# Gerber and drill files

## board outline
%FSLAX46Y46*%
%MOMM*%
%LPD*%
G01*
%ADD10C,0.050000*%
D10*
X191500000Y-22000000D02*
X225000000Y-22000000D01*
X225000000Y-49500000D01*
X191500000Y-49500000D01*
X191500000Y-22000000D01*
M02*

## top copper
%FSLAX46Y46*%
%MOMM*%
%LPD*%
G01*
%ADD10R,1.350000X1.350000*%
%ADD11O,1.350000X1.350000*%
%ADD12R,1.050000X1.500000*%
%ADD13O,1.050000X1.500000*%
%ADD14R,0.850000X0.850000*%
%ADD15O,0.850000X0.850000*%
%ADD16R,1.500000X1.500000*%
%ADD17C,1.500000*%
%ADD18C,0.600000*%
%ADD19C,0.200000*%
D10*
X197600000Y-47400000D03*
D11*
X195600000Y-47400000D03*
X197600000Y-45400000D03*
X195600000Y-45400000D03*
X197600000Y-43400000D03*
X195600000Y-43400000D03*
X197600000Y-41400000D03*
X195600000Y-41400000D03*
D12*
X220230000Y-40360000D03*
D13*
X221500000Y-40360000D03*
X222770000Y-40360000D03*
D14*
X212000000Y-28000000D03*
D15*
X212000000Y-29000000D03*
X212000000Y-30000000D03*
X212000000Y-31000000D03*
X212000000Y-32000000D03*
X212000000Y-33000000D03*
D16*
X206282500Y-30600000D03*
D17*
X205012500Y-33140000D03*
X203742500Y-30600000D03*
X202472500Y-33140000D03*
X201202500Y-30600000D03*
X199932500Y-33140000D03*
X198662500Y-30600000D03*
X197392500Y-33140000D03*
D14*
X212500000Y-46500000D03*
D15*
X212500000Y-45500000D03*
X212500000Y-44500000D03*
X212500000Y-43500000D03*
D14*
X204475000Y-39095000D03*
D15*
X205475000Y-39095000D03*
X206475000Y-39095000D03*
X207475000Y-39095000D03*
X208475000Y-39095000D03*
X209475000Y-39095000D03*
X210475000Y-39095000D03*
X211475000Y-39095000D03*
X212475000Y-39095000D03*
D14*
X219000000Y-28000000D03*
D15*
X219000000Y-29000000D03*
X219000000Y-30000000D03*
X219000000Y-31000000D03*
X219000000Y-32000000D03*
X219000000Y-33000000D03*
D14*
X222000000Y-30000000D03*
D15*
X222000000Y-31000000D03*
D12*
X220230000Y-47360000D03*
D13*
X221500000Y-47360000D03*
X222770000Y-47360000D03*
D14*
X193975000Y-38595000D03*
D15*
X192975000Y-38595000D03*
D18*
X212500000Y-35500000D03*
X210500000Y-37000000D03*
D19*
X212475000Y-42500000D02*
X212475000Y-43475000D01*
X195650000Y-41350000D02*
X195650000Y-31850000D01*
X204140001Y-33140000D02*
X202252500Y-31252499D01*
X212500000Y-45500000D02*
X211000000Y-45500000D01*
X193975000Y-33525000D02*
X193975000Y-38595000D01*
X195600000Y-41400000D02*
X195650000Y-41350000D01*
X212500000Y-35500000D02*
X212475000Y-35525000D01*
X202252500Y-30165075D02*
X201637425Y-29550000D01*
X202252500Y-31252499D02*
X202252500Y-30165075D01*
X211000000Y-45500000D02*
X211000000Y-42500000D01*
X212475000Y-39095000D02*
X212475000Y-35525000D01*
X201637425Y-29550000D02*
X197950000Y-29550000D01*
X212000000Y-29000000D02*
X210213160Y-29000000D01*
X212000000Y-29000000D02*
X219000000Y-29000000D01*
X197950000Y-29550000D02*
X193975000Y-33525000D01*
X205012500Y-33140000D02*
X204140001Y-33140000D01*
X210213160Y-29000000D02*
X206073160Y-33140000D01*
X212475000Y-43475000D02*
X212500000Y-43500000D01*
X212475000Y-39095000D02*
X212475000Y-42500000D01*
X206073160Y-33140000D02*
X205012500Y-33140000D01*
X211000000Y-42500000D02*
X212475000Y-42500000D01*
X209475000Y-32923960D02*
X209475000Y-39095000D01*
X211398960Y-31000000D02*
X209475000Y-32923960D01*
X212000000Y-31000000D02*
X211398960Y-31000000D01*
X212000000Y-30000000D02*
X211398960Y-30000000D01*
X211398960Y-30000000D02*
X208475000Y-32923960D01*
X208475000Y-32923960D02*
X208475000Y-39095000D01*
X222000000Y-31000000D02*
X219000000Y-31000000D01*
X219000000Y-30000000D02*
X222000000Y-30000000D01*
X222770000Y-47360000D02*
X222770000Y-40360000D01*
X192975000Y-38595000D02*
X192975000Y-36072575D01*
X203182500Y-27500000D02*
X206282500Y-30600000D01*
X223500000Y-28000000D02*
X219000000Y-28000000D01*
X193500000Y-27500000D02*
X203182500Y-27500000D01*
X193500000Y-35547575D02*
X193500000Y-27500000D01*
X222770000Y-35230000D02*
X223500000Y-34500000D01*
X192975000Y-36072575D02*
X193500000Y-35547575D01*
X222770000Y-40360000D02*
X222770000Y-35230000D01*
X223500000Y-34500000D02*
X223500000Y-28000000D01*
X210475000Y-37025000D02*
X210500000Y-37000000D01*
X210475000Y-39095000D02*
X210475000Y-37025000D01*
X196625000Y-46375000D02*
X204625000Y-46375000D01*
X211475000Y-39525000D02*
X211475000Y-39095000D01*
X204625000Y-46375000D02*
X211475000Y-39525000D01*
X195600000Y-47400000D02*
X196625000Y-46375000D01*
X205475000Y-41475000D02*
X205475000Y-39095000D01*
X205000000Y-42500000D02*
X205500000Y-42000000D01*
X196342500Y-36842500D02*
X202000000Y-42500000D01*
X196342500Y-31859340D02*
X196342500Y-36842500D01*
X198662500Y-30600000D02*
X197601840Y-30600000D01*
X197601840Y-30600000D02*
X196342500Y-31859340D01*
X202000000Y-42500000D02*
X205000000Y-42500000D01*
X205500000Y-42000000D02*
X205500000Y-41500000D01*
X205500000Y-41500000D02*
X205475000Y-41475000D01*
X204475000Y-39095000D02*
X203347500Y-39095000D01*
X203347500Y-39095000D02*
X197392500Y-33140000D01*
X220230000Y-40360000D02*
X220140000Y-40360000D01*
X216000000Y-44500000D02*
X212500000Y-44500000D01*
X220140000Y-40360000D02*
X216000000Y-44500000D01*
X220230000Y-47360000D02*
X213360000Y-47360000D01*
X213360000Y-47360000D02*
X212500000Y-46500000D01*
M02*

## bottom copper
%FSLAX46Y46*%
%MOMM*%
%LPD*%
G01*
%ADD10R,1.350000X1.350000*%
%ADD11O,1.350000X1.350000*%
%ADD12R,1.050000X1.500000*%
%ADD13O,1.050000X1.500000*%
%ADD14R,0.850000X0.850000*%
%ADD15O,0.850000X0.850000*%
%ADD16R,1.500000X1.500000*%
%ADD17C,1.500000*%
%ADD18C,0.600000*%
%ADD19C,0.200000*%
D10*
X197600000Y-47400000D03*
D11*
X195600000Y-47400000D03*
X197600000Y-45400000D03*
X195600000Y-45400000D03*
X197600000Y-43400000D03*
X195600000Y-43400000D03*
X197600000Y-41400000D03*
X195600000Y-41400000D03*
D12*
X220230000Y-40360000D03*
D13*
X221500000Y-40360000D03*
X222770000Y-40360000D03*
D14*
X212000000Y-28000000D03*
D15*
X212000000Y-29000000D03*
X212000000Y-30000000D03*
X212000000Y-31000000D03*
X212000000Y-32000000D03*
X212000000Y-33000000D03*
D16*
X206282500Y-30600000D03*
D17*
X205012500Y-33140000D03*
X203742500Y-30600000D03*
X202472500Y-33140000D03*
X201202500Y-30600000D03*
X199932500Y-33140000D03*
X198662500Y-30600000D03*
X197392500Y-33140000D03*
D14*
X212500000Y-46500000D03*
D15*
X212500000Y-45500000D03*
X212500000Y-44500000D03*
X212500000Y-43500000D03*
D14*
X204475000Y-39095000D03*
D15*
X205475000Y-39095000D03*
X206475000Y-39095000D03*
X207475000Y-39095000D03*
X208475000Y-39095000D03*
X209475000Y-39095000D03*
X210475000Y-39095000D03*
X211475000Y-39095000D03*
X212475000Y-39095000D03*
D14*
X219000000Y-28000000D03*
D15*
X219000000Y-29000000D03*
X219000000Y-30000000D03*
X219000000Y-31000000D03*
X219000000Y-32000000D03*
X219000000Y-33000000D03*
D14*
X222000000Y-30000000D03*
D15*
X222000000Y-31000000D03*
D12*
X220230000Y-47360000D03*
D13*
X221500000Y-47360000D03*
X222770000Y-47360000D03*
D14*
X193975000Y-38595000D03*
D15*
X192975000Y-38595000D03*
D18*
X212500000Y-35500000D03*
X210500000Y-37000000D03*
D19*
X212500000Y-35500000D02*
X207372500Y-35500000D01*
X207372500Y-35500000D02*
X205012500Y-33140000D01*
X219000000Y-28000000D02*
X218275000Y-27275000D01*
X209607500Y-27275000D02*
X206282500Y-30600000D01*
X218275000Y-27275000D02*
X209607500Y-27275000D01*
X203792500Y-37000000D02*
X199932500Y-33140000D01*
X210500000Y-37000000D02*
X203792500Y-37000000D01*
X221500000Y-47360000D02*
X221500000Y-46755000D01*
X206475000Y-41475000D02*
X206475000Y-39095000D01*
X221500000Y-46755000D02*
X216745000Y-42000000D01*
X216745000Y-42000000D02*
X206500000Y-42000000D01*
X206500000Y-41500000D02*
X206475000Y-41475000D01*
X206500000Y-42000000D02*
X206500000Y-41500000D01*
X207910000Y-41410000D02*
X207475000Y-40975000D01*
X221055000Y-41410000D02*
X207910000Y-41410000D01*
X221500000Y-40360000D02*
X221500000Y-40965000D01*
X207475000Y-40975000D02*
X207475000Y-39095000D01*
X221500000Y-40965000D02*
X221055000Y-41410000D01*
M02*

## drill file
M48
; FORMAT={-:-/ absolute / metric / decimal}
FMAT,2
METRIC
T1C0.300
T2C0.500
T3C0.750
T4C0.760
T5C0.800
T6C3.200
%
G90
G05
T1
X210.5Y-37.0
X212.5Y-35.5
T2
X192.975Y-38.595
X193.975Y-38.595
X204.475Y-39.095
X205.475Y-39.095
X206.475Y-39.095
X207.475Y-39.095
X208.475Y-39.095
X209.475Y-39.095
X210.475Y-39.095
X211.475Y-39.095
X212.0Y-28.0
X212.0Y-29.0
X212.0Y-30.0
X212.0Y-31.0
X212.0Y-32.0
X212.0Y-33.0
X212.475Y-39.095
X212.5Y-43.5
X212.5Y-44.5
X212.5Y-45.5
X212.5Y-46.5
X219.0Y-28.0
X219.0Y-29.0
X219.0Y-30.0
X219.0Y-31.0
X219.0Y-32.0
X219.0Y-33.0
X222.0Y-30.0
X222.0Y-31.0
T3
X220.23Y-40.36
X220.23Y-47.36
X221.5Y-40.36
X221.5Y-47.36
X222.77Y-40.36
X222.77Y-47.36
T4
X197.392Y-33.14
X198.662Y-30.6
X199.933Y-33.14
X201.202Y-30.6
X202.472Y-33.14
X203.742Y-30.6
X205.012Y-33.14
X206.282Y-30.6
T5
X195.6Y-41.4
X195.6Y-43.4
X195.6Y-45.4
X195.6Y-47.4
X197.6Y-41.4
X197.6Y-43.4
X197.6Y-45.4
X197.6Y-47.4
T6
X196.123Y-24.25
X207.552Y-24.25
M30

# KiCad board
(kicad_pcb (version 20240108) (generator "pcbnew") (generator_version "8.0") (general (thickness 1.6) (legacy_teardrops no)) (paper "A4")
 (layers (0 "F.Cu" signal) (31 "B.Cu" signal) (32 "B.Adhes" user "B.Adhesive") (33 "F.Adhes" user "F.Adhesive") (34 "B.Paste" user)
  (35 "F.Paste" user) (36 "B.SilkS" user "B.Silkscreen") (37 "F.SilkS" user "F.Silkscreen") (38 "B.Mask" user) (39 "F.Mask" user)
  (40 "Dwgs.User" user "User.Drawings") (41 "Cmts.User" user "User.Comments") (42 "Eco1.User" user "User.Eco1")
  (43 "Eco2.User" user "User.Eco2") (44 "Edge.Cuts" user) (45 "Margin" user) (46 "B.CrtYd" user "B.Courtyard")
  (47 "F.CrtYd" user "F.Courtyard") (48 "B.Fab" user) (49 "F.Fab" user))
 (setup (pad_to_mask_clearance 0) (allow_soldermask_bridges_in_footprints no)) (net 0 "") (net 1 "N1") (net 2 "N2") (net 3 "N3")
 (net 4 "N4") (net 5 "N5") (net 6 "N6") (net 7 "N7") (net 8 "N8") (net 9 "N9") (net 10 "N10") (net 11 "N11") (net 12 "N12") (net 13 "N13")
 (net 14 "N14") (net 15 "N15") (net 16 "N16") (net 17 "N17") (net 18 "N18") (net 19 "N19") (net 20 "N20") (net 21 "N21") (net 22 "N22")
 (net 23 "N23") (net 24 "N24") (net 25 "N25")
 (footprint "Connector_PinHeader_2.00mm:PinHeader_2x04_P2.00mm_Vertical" (layer "F.Cu") (at 197.6 47.4 180)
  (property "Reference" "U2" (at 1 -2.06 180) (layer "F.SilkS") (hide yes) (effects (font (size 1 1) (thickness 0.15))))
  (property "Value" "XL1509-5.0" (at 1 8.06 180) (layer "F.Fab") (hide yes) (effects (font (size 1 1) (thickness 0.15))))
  (pad "1" thru_hole rect (at 0 0 180) (size 1.35 1.35) (drill 0.8) (layers "*.Cu" "*.Mask") (remove_unused_layers no) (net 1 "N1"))
  (pad "2" thru_hole oval (at 2 0 180) (size 1.35 1.35) (drill 0.8) (layers "*.Cu" "*.Mask") (remove_unused_layers no) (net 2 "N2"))
  (pad "3" thru_hole oval (at 0 2 180) (size 1.35 1.35) (drill 0.8) (layers "*.Cu" "*.Mask") (remove_unused_layers no) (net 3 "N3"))
  (pad "4" thru_hole oval (at 2 2 180) (size 1.35 1.35) (drill 0.8) (layers "*.Cu" "*.Mask") (remove_unused_layers no) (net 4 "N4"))
  (pad "5" thru_hole oval (at 0 4 180) (size 1.35 1.35) (drill 0.8) (layers "*.Cu" "*.Mask") (remove_unused_layers no) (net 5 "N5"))
  (pad "6" thru_hole oval (at 2 4 180) (size 1.35 1.35) (drill 0.8) (layers "*.Cu" "*.Mask") (remove_unused_layers no) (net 5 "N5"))
  (pad "7" thru_hole oval (at 0 6 180) (size 1.35 1.35) (drill 0.8) (layers "*.Cu" "*.Mask") (remove_unused_layers no) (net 5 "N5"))
  (pad "8" thru_hole oval (at 2 6 180) (size 1.35 1.35) (drill 0.8) (layers "*.Cu" "*.Mask") (remove_unused_layers no) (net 5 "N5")))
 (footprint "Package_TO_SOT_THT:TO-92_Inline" (layer "F.Cu") (at 220.23 40.36)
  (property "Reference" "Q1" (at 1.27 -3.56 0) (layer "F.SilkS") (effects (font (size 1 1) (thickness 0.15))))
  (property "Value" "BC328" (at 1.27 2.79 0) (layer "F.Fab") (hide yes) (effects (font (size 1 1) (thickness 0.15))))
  (pad "1" thru_hole rect (at 0 0) (size 1.05 1.5) (drill 0.75) (layers "*.Cu" "*.Mask") (remove_unused_layers no) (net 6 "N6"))
  (pad "2" thru_hole oval (at 1.27 0) (size 1.05 1.5) (drill 0.75) (layers "*.Cu" "*.Mask") (remove_unused_layers no) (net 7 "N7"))
  (pad "3" thru_hole oval (at 2.54 0) (size 1.05 1.5) (drill 0.75) (layers "*.Cu" "*.Mask") (remove_unused_layers no) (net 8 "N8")))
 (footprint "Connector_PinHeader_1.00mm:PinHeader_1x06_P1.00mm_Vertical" (layer "F.Cu") (at 212 28)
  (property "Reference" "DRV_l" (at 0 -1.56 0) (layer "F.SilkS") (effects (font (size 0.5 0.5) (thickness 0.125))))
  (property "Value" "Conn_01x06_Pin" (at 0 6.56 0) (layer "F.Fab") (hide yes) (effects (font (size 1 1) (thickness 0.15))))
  (pad "1" thru_hole rect (at 0 0) (size 0.85 0.85) (drill 0.5) (layers "*.Cu" "*.Mask") (remove_unused_layers no) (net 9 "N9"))
  (pad "2" thru_hole oval (at 0 1) (size 0.85 0.85) (drill 0.5) (layers "*.Cu" "*.Mask") (remove_unused_layers no) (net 5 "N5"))
  (pad "3" thru_hole oval (at 0 2) (size 0.85 0.85) (drill 0.5) (layers "*.Cu" "*.Mask") (remove_unused_layers no) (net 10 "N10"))
  (pad "4" thru_hole oval (at 0 3) (size 0.85 0.85) (drill 0.5) (layers "*.Cu" "*.Mask") (remove_unused_layers no) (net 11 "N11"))
  (pad "5" thru_hole oval (at 0 4) (size 0.85 0.85) (drill 0.5) (layers "*.Cu" "*.Mask") (remove_unused_layers no) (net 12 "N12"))
  (pad "6" thru_hole oval (at 0 5) (size 0.85 0.85) (drill 0.5) (layers "*.Cu" "*.Mask") (remove_unused_layers no) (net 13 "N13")))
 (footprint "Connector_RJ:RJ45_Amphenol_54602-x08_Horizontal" (layer "F.Cu") (at 206.2825 30.6 180)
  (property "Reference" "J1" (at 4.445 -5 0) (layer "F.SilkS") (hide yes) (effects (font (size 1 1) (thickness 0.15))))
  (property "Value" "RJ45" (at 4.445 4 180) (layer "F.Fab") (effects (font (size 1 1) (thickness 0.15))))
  (pad "" np_thru_hole circle (at -1.27 6.35 180) (size 3.2 3.2) (drill 3.2) (layers "*.Cu" "*.Mask"))
  (pad "" np_thru_hole circle (at 10.16 6.35 180) (size 3.2 3.2) (drill 3.2) (layers "*.Cu" "*.Mask"))
  (pad "1" thru_hole rect (at 0 0 180) (size 1.5 1.5) (drill 0.76) (layers "*.Cu" "*.Mask") (remove_unused_layers no) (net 8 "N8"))
  (pad "2" thru_hole circle (at 1.27 -2.54 180) (size 1.5 1.5) (drill 0.76) (layers "*.Cu" "*.Mask") (remove_unused_layers no) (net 5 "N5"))
  (pad "3" thru_hole circle (at 2.54 0 180) (size 1.5 1.5) (drill 0.76) (layers "*.Cu" "*.Mask") (remove_unused_layers no) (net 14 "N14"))
  (pad "4" thru_hole circle (at 3.81 -2.54 180) (size 1.5 1.5) (drill 0.76) (layers "*.Cu" "*.Mask") (remove_unused_layers no)
   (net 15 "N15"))
  (pad "5" thru_hole circle (at 5.08 0 180) (size 1.5 1.5) (drill 0.76) (layers "*.Cu" "*.Mask") (remove_unused_layers no) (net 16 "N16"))
  (pad "6" thru_hole circle (at 6.35 -2.54 180) (size 1.5 1.5) (drill 0.76) (layers "*.Cu" "*.Mask") (remove_unused_layers no)
   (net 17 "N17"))
  (pad "7" thru_hole circle (at 7.62 0 180) (size 1.5 1.5) (drill 0.76) (layers "*.Cu" "*.Mask") (remove_unused_layers no) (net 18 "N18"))
  (pad "8" thru_hole circle (at 8.89 -2.54 180) (size 1.5 1.5) (drill 0.76) (layers "*.Cu" "*.Mask") (remove_unused_layers no)
   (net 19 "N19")))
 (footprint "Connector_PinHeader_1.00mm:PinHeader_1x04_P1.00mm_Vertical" (layer "F.Cu") (at 212.5 46.5 180)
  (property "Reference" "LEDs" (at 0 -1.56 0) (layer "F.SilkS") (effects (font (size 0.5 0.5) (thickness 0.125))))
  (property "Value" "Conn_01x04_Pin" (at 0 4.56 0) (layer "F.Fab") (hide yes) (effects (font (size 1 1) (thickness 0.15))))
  (pad "1" thru_hole rect (at 0 0 180) (size 0.85 0.85) (drill 0.5) (layers "*.Cu" "*.Mask") (remove_unused_layers no) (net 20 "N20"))
  (pad "2" thru_hole oval (at 0 1 180) (size 0.85 0.85) (drill 0.5) (layers "*.Cu" "*.Mask") (remove_unused_layers no) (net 5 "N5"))
  (pad "3" thru_hole oval (at 0 2 180) (size 0.85 0.85) (drill 0.5) (layers "*.Cu" "*.Mask") (remove_unused_layers no) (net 6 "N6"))
  (pad "4" thru_hole oval (at 0 3 180) (size 0.85 0.85) (drill 0.5) (layers "*.Cu" "*.Mask") (remove_unused_layers no) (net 5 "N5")))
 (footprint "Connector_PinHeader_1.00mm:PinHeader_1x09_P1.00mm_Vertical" (layer "F.Cu") (at 204.475 39.095 90)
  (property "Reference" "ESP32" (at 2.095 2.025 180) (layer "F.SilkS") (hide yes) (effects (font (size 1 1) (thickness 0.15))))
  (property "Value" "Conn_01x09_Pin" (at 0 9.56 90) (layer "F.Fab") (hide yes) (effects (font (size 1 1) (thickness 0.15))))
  (pad "1" thru_hole rect (at 0 0 90) (size 0.85 0.85) (drill 0.5) (layers "*.Cu" "*.Mask") (remove_unused_layers no) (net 19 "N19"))
  (pad "2" thru_hole oval (at 0 1 90) (size 0.85 0.85) (drill 0.5) (layers "*.Cu" "*.Mask") (remove_unused_layers no) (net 18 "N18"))
  (pad "3" thru_hole oval (at 0 2 90) (size 0.85 0.85) (drill 0.5) (layers "*.Cu" "*.Mask") (remove_unused_layers no) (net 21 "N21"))
  (pad "4" thru_hole oval (at 0 3 90) (size 0.85 0.85) (drill 0.5) (layers "*.Cu" "*.Mask") (remove_unused_layers no) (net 7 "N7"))
  (pad "5" thru_hole oval (at 0 4 90) (size 0.85 0.85) (drill 0.5) (layers "*.Cu" "*.Mask") (remove_unused_layers no) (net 10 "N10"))
  (pad "6" thru_hole oval (at 0 5 90) (size 0.85 0.85) (drill 0.5) (layers "*.Cu" "*.Mask") (remove_unused_layers no) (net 11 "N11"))
  (pad "7" thru_hole oval (at 0 6 90) (size 0.85 0.85) (drill 0.5) (layers "*.Cu" "*.Mask") (remove_unused_layers no) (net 17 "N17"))
  (pad "8" thru_hole oval (at 0 7 90) (size 0.85 0.85) (drill 0.5) (layers "*.Cu" "*.Mask") (remove_unused_layers no) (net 2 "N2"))
  (pad "9" thru_hole oval (at 0 8 90) (size 0.85 0.85) (drill 0.5) (layers "*.Cu" "*.Mask") (remove_unused_layers no) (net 5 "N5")))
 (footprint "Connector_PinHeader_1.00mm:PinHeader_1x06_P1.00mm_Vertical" (layer "F.Cu") (at 219 28)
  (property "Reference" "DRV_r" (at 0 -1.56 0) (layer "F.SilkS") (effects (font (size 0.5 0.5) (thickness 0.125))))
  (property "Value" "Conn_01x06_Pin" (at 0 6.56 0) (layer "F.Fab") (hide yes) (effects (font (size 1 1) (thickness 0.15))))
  (pad "1" thru_hole rect (at 0 0) (size 0.85 0.85) (drill 0.5) (layers "*.Cu" "*.Mask") (remove_unused_layers no) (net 8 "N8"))
  (pad "2" thru_hole oval (at 0 1) (size 0.85 0.85) (drill 0.5) (layers "*.Cu" "*.Mask") (remove_unused_layers no) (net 5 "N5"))
  (pad "3" thru_hole oval (at 0 2) (size 0.85 0.85) (drill 0.5) (layers "*.Cu" "*.Mask") (remove_unused_layers no) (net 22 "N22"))
  (pad "4" thru_hole oval (at 0 3) (size 0.85 0.85) (drill 0.5) (layers "*.Cu" "*.Mask") (remove_unused_layers no) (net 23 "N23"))
  (pad "5" thru_hole oval (at 0 4) (size 0.85 0.85) (drill 0.5) (layers "*.Cu" "*.Mask") (remove_unused_layers no) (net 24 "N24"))
  (pad "6" thru_hole oval (at 0 5) (size 0.85 0.85) (drill 0.5) (layers "*.Cu" "*.Mask") (remove_unused_layers no) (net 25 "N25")))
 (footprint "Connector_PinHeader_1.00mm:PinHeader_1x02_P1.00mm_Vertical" (layer "F.Cu") (at 222 30)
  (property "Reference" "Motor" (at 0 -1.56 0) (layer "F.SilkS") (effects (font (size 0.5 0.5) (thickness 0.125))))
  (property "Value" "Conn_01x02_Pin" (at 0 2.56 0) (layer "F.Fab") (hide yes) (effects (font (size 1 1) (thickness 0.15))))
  (pad "1" thru_hole rect (at 0 0) (size 0.85 0.85) (drill 0.5) (layers "*.Cu" "*.Mask") (remove_unused_layers no) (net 22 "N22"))
  (pad "2" thru_hole oval (at 0 1) (size 0.85 0.85) (drill 0.5) (layers "*.Cu" "*.Mask") (remove_unused_layers no) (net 23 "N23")))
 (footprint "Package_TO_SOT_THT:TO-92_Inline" (layer "F.Cu") (at 220.23 47.36)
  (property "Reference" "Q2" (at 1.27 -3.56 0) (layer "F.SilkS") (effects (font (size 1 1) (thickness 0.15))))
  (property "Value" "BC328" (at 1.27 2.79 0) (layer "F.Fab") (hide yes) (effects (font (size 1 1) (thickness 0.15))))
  (pad "1" thru_hole rect (at 0 0) (size 1.05 1.5) (drill 0.75) (layers "*.Cu" "*.Mask") (remove_unused_layers no) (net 20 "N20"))
  (pad "2" thru_hole oval (at 1.27 0) (size 1.05 1.5) (drill 0.75) (layers "*.Cu" "*.Mask") (remove_unused_layers no) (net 21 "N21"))
  (pad "3" thru_hole oval (at 2.54 0) (size 1.05 1.5) (drill 0.75) (layers "*.Cu" "*.Mask") (remove_unused_layers no) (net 8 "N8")))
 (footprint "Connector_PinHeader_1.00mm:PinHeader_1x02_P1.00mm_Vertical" (layer "F.Cu") (at 193.975 38.595 -90)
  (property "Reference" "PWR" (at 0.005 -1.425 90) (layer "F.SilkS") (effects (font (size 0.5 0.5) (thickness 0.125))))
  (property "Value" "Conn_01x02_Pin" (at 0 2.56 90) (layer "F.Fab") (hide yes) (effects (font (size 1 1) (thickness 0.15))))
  (pad "1" thru_hole rect (at 0 0 270) (size 0.85 0.85) (drill 0.5) (layers "*.Cu" "*.Mask") (remove_unused_layers no) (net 5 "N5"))
  (pad "2" thru_hole oval (at 0 1 270) (size 0.85 0.85) (drill 0.5) (layers "*.Cu" "*.Mask") (remove_unused_layers no) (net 8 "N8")))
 (gr_rect (start 191.5 22) (end 225 49.5) (stroke (width 0.05) (type default)) (fill none) (layer "Edge.Cuts"))
 (segment (start 212.475 42.5) (end 212.475 43.475) (width 0.2) (layer "F.Cu") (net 5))
 (segment (start 195.65 41.35) (end 195.65 31.85) (width 0.2) (layer "F.Cu") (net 5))
 (segment (start 204.140001 33.14) (end 202.2525 31.252499) (width 0.2) (layer "F.Cu") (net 5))
 (segment (start 212.5 45.5) (end 211 45.5) (width 0.2) (layer "F.Cu") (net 5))
 (segment (start 193.975 33.525) (end 193.975 38.595) (width 0.2) (layer "F.Cu") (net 5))
 (segment (start 195.6 41.4) (end 195.65 41.35) (width 0.2) (layer "F.Cu") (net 5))
 (segment (start 212.5 35.5) (end 212.475 35.525) (width 0.2) (layer "F.Cu") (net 5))
 (segment (start 202.2525 30.165075) (end 201.637425 29.55) (width 0.2) (layer "F.Cu") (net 5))
 (segment (start 202.2525 31.252499) (end 202.2525 30.165075) (width 0.2) (layer "F.Cu") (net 5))
 (segment (start 211 45.5) (end 211 42.5) (width 0.2) (layer "F.Cu") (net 5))
 (segment (start 212.475 39.095) (end 212.475 35.525) (width 0.2) (layer "F.Cu") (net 5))
 (segment (start 201.637425 29.55) (end 197.95 29.55) (width 0.2) (layer "F.Cu") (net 5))
 (segment (start 212 29) (end 210.21316 29) (width 0.2) (layer "F.Cu") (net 5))
 (segment (start 212 29) (end 219 29) (width 0.2) (layer "F.Cu") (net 5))
 (segment (start 197.95 29.55) (end 193.975 33.525) (width 0.2) (layer "F.Cu") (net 5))
 (segment (start 205.0125 33.14) (end 204.140001 33.14) (width 0.2) (layer "F.Cu") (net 5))
 (segment (start 210.21316 29) (end 206.07316 33.14) (width 0.2) (layer "F.Cu") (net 5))
 (segment (start 212.475 43.475) (end 212.5 43.5) (width 0.2) (layer "F.Cu") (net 5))
 (segment (start 212.475 39.095) (end 212.475 42.5) (width 0.2) (layer "F.Cu") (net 5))
 (segment (start 206.07316 33.14) (end 205.0125 33.14) (width 0.2) (layer "F.Cu") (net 5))
 (segment (start 211 42.5) (end 212.475 42.5) (width 0.2) (layer "F.Cu") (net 5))
 (via (at 212.5 35.5) (size 0.6) (drill 0.3) (layers "F.Cu" "B.Cu") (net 5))
 (segment (start 212.5 35.5) (end 207.3725 35.5) (width 0.2) (layer "B.Cu") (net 5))
 (segment (start 207.3725 35.5) (end 205.0125 33.14) (width 0.2) (layer "B.Cu") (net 5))
 (segment (start 209.475 32.92396) (end 209.475 39.095) (width 0.2) (layer "F.Cu") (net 11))
 (segment (start 211.39896 31) (end 209.475 32.92396) (width 0.2) (layer "F.Cu") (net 11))
 (segment (start 212 31) (end 211.39896 31) (width 0.2) (layer "F.Cu") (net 11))
 (segment (start 212 30) (end 211.39896 30) (width 0.2) (layer "F.Cu") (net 10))
 (segment (start 211.39896 30) (end 208.475 32.92396) (width 0.2) (layer "F.Cu") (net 10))
 (segment (start 208.475 32.92396) (end 208.475 39.095) (width 0.2) (layer "F.Cu") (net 10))
 (segment (start 222 31) (end 219 31) (width 0.2) (layer "F.Cu") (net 23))
 (segment (start 219 30) (end 222 30) (width 0.2) (layer "F.Cu") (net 22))
 (segment (start 222.77 47.36) (end 222.77 40.36) (width 0.2) (layer "F.Cu") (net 8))
 (segment (start 192.975 38.595) (end 192.975 36.072575) (width 0.2) (layer "F.Cu") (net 8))
 (segment (start 203.1825 27.5) (end 206.2825 30.6) (width 0.2) (layer "F.Cu") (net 8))
 (segment (start 223.5 28) (end 219 28) (width 0.2) (layer "F.Cu") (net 8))
 (segment (start 193.5 27.5) (end 203.1825 27.5) (width 0.2) (layer "F.Cu") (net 8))
 (segment (start 193.5 35.547575) (end 193.5 27.5) (width 0.2) (layer "F.Cu") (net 8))
 (segment (start 222.77 35.23) (end 223.5 34.5) (width 0.2) (layer "F.Cu") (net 8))
 (segment (start 192.975 36.072575) (end 193.5 35.547575) (width 0.2) (layer "F.Cu") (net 8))
 (segment (start 222.77 40.36) (end 222.77 35.23) (width 0.2) (layer "F.Cu") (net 8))
 (segment (start 223.5 34.5) (end 223.5 28) (width 0.2) (layer "F.Cu") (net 8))
 (segment (start 219 28) (end 218.275 27.275) (width 0.2) (layer "B.Cu") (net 8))
 (segment (start 209.6075 27.275) (end 206.2825 30.6) (width 0.2) (layer "B.Cu") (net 8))
 (segment (start 218.275 27.275) (end 209.6075 27.275) (width 0.2) (layer "B.Cu") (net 8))
 (segment (start 210.475 37.025) (end 210.5 37) (width 0.2) (layer "F.Cu") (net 17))
 (segment (start 210.475 39.095) (end 210.475 37.025) (width 0.2) (layer "F.Cu") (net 17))
 (via (at 210.5 37) (size 0.6) (drill 0.3) (layers "F.Cu" "B.Cu") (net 17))
 (segment (start 203.7925 37) (end 199.9325 33.14) (width 0.2) (layer "B.Cu") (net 17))
 (segment (start 210.5 37) (end 203.7925 37) (width 0.2) (layer "B.Cu") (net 17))
 (segment (start 196.625 46.375) (end 204.625 46.375) (width 0.2) (layer "F.Cu") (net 2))
 (segment (start 211.475 39.525) (end 211.475 39.095) (width 0.2) (layer "F.Cu") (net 2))
 (segment (start 204.625 46.375) (end 211.475 39.525) (width 0.2) (layer "F.Cu") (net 2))
 (segment (start 195.6 47.4) (end 196.625 46.375) (width 0.2) (layer "F.Cu") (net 2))
 (segment (start 221.5 47.36) (end 221.5 46.755) (width 0.2) (layer "B.Cu") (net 21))
 (segment (start 206.475 41.475) (end 206.475 39.095) (width 0.2) (layer "B.Cu") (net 21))
 (segment (start 221.5 46.755) (end 216.745 42) (width 0.2) (layer "B.Cu") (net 21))
 (segment (start 216.745 42) (end 206.5 42) (width 0.2) (layer "B.Cu") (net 21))
 (segment (start 206.5 41.5) (end 206.475 41.475) (width 0.2) (layer "B.Cu") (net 21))
 (segment (start 206.5 42) (end 206.5 41.5) (width 0.2) (layer "B.Cu") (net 21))
 (segment (start 207.91 41.41) (end 207.475 40.975) (width 0.2) (layer "B.Cu") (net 7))
 (segment (start 221.055 41.41) (end 207.91 41.41) (width 0.2) (layer "B.Cu") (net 7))
 (segment (start 221.5 40.36) (end 221.5 40.965) (width 0.2) (layer "B.Cu") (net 7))
 (segment (start 207.475 40.975) (end 207.475 39.095) (width 0.2) (layer "B.Cu") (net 7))
 (segment (start 221.5 40.965) (end 221.055 41.41) (width 0.2) (layer "B.Cu") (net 7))
 (segment (start 205.475 41.475) (end 205.475 39.095) (width 0.2) (layer "F.Cu") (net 18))
 (segment (start 205 42.5) (end 205.5 42) (width 0.2) (layer "F.Cu") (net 18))
 (segment (start 196.3425 36.8425) (end 202 42.5) (width 0.2) (layer "F.Cu") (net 18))
 (segment (start 196.3425 31.85934) (end 196.3425 36.8425) (width 0.2) (layer "F.Cu") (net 18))
 (segment (start 198.6625 30.6) (end 197.60184 30.6) (width 0.2) (layer "F.Cu") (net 18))
 (segment (start 197.60184 30.6) (end 196.3425 31.85934) (width 0.2) (layer "F.Cu") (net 18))
 (segment (start 202 42.5) (end 205 42.5) (width 0.2) (layer "F.Cu") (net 18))
 (segment (start 205.5 42) (end 205.5 41.5) (width 0.2) (layer "F.Cu") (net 18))
 (segment (start 205.5 41.5) (end 205.475 41.475) (width 0.2) (layer "F.Cu") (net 18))
 (segment (start 204.475 39.095) (end 203.3475 39.095) (width 0.2) (layer "F.Cu") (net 19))
 (segment (start 203.3475 39.095) (end 197.3925 33.14) (width 0.2) (layer "F.Cu") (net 19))
 (segment (start 220.23 40.36) (end 220.14 40.36) (width 0.2) (layer "F.Cu") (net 6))
 (segment (start 216 44.5) (end 212.5 44.5) (width 0.2) (layer "F.Cu") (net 6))
 (segment (start 220.14 40.36) (end 216 44.5) (width 0.2) (layer "F.Cu") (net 6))
 (segment (start 220.23 47.36) (end 213.36 47.36) (width 0.2) (layer "F.Cu") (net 20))
 (segment (start 213.36 47.36) (end 212.5 46.5) (width 0.2) (layer "F.Cu") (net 20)))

